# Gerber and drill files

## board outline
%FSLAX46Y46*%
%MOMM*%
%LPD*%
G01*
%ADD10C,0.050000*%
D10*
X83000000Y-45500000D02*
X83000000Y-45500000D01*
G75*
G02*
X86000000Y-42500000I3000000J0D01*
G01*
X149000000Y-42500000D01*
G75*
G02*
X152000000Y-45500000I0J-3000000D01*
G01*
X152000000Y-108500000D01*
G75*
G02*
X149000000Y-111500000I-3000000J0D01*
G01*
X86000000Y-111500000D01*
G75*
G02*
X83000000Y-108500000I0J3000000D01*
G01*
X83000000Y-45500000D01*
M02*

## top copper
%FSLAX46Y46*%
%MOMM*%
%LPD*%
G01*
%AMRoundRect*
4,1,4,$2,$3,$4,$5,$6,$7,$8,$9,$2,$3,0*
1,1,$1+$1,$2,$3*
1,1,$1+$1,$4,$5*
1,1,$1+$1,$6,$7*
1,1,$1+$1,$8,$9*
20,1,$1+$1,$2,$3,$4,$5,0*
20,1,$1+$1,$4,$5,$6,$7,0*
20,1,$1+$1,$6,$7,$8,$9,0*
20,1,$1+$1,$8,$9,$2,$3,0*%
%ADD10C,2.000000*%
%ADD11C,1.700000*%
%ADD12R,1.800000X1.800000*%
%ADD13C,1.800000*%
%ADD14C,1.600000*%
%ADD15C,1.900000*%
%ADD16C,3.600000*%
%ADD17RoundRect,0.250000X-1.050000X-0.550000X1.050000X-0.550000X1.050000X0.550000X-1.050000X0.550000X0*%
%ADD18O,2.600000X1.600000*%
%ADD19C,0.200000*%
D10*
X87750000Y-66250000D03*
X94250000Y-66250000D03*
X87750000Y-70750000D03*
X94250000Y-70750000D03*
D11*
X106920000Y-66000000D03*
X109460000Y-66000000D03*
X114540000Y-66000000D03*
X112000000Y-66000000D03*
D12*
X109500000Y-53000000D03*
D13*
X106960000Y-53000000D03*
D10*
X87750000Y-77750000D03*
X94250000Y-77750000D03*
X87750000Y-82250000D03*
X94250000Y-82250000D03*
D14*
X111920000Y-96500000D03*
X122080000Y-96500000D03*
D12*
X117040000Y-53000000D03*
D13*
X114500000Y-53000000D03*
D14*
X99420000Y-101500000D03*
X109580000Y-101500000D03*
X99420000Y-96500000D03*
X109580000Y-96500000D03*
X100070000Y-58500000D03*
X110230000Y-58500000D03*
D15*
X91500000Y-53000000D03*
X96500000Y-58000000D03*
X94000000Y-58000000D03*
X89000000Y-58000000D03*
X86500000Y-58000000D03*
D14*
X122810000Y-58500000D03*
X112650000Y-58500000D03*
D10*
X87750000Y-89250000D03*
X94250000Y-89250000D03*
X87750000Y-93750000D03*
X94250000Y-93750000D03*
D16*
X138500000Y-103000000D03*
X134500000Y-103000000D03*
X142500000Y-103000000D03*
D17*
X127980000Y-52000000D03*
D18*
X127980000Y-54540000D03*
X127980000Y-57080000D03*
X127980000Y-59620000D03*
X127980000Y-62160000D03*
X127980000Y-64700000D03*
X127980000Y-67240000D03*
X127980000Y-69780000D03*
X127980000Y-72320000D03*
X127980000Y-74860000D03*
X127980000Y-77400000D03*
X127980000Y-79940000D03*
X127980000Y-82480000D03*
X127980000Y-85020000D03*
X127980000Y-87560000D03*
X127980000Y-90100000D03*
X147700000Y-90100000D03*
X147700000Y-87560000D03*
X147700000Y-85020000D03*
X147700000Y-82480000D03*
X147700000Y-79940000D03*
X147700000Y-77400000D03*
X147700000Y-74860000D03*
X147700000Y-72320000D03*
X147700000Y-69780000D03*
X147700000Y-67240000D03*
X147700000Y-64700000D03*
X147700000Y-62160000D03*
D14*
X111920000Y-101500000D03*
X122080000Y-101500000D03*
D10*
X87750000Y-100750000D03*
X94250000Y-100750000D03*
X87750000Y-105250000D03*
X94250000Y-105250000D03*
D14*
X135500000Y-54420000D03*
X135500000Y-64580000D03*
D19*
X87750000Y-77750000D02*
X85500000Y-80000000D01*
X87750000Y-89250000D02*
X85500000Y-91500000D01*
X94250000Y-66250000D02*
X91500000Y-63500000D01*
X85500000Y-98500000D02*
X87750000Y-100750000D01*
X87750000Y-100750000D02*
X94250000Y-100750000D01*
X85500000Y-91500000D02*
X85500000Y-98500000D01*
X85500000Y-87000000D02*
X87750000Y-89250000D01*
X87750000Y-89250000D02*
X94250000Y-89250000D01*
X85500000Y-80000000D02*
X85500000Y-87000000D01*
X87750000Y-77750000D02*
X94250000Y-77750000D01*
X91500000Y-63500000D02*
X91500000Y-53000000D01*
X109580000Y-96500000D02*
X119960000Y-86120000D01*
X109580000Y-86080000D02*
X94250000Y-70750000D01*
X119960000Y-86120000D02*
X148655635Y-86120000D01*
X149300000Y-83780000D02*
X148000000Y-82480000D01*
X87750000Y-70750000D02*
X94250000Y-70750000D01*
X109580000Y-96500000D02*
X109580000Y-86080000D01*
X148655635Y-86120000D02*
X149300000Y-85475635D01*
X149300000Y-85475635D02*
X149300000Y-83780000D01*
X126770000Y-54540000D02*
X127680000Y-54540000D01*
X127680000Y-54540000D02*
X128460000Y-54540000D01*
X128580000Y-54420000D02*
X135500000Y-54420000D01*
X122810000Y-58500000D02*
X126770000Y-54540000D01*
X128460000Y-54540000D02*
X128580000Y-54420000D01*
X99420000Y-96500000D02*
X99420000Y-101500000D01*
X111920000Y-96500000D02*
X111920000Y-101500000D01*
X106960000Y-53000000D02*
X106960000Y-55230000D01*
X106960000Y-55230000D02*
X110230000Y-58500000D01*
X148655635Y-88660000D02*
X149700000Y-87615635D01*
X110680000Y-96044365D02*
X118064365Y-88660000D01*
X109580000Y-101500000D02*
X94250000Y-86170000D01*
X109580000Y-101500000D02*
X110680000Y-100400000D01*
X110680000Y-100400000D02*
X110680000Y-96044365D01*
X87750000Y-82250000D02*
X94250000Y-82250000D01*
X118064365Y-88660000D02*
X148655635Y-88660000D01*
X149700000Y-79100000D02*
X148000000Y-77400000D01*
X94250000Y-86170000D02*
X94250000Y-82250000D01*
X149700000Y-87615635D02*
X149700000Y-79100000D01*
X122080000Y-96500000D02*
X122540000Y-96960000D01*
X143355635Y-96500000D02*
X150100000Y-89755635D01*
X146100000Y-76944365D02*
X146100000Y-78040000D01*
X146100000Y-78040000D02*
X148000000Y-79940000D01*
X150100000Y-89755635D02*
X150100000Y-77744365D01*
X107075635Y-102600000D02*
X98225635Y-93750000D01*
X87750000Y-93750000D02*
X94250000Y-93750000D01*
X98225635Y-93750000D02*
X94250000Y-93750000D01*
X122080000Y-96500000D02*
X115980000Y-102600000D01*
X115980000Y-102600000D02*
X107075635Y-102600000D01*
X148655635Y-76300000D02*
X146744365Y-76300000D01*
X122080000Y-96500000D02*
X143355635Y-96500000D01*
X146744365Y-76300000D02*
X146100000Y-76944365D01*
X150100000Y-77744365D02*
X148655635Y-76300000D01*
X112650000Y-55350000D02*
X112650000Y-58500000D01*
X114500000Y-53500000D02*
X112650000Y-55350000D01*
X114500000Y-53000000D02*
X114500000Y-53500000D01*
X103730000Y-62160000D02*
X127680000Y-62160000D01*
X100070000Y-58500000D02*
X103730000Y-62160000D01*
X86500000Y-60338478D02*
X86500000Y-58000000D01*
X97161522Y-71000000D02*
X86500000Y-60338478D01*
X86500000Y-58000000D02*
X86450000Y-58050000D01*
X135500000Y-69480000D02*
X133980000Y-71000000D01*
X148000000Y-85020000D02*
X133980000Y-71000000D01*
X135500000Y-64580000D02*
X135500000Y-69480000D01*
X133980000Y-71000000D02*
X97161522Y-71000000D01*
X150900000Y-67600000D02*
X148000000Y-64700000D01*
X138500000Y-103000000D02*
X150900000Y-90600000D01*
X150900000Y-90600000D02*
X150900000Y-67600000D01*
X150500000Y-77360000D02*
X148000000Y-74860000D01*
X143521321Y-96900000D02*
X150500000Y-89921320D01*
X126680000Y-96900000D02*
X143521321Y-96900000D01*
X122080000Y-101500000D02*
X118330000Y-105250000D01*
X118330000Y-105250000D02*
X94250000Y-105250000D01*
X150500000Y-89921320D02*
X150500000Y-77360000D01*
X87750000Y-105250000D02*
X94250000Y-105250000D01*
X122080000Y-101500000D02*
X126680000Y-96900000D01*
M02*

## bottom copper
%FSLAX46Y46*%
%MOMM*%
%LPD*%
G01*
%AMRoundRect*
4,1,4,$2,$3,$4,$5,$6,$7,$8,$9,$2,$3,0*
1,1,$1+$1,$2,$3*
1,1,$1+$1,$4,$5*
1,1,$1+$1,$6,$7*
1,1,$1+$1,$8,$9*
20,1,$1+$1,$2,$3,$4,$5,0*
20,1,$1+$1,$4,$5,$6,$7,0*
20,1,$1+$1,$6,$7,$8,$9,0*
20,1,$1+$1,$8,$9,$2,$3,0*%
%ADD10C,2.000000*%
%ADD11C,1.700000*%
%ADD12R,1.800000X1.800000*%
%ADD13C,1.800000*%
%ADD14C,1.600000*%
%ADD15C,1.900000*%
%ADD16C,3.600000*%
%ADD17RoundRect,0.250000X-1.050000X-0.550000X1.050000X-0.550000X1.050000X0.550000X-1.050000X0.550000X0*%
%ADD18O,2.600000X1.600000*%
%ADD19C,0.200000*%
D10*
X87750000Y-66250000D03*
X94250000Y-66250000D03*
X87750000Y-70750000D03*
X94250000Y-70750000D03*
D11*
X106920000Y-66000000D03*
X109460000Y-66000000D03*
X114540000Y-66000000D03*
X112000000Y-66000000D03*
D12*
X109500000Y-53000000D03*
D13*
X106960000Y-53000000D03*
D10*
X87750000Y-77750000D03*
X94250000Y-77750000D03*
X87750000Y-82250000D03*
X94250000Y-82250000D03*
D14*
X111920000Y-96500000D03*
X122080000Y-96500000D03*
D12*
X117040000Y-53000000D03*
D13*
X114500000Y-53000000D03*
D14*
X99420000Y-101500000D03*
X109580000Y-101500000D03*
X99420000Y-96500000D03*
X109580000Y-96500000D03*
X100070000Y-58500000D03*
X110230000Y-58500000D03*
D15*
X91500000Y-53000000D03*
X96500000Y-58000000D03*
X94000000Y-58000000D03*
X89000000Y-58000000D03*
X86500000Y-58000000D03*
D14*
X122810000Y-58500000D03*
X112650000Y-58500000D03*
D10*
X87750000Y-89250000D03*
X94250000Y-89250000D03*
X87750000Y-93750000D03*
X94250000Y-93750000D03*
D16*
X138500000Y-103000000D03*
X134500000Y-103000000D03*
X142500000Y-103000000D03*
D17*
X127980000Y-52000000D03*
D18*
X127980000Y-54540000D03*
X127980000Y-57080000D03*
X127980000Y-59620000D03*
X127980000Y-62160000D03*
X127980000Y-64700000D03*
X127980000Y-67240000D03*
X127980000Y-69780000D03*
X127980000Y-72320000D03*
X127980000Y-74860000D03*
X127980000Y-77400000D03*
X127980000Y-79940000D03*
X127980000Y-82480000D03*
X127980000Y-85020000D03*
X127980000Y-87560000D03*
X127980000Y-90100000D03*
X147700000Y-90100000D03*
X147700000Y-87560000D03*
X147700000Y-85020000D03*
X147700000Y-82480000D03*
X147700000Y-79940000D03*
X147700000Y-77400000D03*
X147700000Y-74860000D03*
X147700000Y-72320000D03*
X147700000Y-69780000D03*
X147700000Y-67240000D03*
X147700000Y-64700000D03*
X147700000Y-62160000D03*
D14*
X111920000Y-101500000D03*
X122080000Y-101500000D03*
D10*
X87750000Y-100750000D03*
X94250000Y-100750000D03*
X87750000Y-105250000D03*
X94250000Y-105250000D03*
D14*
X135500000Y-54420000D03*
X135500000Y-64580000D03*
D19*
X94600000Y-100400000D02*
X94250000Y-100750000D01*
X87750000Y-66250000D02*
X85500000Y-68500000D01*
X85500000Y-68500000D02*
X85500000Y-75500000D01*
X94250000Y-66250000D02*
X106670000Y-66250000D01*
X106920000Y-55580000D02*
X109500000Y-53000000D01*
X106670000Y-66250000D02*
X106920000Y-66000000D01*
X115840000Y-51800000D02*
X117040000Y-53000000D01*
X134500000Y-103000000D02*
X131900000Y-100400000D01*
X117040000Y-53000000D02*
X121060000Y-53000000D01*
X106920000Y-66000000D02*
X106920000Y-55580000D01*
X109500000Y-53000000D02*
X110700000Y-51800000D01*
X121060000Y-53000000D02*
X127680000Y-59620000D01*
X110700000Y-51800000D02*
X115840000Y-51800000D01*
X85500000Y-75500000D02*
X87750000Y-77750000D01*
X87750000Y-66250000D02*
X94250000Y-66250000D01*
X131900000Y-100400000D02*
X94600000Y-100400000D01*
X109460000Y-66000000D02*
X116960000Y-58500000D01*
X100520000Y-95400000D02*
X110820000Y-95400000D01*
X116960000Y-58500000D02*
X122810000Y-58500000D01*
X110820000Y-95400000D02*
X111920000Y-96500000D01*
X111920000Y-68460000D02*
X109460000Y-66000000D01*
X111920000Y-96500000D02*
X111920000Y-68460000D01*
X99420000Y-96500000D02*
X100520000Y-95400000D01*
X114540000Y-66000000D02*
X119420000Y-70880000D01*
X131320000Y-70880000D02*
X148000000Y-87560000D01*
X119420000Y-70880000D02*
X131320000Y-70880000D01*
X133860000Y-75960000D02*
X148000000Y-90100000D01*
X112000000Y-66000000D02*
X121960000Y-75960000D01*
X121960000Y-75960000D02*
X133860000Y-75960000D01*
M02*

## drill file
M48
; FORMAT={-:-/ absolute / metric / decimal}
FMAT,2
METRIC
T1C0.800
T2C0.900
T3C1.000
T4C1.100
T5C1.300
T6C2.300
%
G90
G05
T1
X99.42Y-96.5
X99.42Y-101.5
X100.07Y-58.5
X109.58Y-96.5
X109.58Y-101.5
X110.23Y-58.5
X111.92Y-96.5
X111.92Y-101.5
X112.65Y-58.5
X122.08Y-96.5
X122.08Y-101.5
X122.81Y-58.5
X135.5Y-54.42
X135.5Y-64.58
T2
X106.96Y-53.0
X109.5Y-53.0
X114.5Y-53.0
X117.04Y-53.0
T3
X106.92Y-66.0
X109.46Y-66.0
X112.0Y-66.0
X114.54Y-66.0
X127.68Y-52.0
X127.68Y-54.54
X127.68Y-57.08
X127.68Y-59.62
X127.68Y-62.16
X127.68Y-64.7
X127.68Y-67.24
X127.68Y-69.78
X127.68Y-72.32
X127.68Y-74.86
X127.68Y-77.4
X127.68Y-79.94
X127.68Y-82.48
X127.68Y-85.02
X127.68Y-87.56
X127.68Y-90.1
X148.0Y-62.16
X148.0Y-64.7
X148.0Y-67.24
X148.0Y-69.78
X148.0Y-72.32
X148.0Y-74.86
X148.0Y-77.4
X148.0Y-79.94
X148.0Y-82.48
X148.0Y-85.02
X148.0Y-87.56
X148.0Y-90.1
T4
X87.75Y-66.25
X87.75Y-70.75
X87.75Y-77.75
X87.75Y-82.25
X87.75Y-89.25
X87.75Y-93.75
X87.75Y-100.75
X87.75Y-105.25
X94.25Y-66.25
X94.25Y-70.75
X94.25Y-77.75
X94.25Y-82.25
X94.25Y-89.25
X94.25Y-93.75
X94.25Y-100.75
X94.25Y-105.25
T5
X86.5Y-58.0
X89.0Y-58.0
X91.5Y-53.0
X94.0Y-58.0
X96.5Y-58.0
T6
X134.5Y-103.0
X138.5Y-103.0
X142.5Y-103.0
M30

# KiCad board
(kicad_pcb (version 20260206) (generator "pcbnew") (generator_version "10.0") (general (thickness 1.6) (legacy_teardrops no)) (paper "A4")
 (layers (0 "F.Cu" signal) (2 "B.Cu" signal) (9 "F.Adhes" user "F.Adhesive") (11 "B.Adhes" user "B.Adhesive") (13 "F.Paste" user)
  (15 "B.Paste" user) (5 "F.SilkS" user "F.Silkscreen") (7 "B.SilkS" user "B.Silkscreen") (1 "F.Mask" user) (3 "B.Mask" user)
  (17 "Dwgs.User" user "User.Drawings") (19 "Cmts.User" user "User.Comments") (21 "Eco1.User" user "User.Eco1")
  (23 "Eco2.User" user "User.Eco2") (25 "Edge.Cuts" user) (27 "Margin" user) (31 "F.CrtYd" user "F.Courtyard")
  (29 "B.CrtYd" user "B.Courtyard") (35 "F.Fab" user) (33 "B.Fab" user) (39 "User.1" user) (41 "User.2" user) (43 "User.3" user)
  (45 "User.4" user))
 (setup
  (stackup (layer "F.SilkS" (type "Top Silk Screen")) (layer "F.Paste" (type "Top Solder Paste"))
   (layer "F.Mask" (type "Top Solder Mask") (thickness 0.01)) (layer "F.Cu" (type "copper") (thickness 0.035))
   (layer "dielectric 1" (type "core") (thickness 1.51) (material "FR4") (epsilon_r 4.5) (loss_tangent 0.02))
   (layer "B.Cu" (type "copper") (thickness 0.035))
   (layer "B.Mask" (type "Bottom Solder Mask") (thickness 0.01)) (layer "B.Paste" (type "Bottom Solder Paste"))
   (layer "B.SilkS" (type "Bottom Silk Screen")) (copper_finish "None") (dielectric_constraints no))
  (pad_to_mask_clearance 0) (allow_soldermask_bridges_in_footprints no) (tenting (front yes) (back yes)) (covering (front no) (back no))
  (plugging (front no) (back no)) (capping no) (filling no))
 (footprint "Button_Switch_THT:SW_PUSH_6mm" (layer "F.Cu") (at 87.75 66.25)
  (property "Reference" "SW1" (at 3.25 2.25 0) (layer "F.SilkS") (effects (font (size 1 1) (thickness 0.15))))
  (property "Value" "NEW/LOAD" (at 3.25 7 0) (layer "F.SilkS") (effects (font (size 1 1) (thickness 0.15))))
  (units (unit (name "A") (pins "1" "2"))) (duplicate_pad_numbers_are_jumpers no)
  (pad "1" thru_hole circle (at 0 0 90) (size 2 2) (drill 1.1) (layers "*.Cu" "*.Mask") (remove_unused_layers no) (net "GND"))
  (pad "1" thru_hole circle (at 6.5 0 90) (size 2 2) (drill 1.1) (layers "*.Cu" "*.Mask") (remove_unused_layers no) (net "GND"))
  (pad "2" thru_hole circle (at 0 4.5 90) (size 2 2) (drill 1.1) (layers "*.Cu" "*.Mask") (remove_unused_layers no) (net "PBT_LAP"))
  (pad "2" thru_hole circle (at 6.5 4.5 90) (size 2 2) (drill 1.1) (layers "*.Cu" "*.Mask") (remove_unused_layers no) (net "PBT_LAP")))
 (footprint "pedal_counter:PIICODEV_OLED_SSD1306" (layer "F.Cu") (at 110.73 78)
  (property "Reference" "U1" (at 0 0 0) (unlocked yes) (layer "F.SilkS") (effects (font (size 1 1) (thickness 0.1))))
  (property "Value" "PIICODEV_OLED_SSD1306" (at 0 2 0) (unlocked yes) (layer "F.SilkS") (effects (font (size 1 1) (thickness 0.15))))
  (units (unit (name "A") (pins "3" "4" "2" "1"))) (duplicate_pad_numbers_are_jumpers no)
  (pad "1" thru_hole circle (at -3.81 -12) (size 1.7 1.7) (drill 1) (layers "*.Cu" "*.Mask") (remove_unused_layers no) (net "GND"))
  (pad "2" thru_hole circle (at -1.27 -12) (size 1.7 1.7) (drill 1) (layers "*.Cu" "*.Mask") (remove_unused_layers no) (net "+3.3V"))
  (pad "3" thru_hole circle (at 3.81 -12) (size 1.7 1.7) (drill 1) (layers "*.Cu" "*.Mask") (remove_unused_layers no) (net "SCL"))
  (pad "4" thru_hole circle (at 1.27 -12) (size 1.7 1.7) (drill 1) (layers "*.Cu" "*.Mask") (remove_unused_layers no) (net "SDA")))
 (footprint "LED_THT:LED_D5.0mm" (layer "F.Cu") (at 109.5 53 180)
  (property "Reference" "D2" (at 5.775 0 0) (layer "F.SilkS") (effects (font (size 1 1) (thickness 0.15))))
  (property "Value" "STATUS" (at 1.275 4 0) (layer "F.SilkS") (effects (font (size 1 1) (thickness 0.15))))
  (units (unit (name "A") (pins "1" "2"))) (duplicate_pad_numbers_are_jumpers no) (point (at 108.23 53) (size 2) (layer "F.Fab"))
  (pad "1" thru_hole rect (at 0 0 180) (size 1.8 1.8) (drill 0.9) (layers "*.Cu" "*.Mask") (remove_unused_layers no) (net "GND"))
  (pad "2" thru_hole circle (at 2.54 0 180) (size 1.8 1.8) (drill 0.9) (layers "*.Cu" "*.Mask") (remove_unused_layers no) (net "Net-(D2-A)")))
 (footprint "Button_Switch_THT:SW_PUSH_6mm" (layer "F.Cu") (at 87.75 77.75)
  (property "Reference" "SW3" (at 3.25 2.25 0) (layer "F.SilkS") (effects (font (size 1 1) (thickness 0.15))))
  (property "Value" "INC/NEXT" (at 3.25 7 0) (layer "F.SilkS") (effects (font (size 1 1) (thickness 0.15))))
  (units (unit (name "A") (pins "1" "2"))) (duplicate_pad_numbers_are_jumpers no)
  (pad "1" thru_hole circle (at 0 0 90) (size 2 2) (drill 1.1) (layers "*.Cu" "*.Mask") (remove_unused_layers no) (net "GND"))
  (pad "1" thru_hole circle (at 6.5 0 90) (size 2 2) (drill 1.1) (layers "*.Cu" "*.Mask") (remove_unused_layers no) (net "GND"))
  (pad "2" thru_hole circle (at 0 4.5 90) (size 2 2) (drill 1.1) (layers "*.Cu" "*.Mask") (remove_unused_layers no) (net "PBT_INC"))
  (pad "2" thru_hole circle (at 6.5 4.5 90) (size 2 2) (drill 1.1) (layers "*.Cu" "*.Mask") (remove_unused_layers no) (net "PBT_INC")))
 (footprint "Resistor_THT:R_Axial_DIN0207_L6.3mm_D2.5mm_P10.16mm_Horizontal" (layer "F.Cu") (at 111.92 96.5)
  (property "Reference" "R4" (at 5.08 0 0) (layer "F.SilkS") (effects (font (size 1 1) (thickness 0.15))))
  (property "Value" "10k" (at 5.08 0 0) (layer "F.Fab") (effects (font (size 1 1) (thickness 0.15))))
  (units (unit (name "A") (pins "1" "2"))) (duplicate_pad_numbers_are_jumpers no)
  (pad "1" thru_hole circle (at 0 0) (size 1.6 1.6) (drill 0.8) (layers "*.Cu" "*.Mask") (remove_unused_layers no) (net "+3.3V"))
  (pad "2" thru_hole circle (at 10.16 0) (size 1.6 1.6) (drill 0.8) (layers "*.Cu" "*.Mask") (remove_unused_layers no) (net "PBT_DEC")))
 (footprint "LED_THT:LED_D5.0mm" (layer "F.Cu") (at 117.04 53 180)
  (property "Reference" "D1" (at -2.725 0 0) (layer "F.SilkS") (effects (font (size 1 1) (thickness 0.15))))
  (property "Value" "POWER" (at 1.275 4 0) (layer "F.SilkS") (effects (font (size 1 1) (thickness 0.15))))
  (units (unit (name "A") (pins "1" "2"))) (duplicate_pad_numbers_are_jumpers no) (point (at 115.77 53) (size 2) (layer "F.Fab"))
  (pad "1" thru_hole rect (at 0 0 180) (size 1.8 1.8) (drill 0.9) (layers "*.Cu" "*.Mask") (remove_unused_layers no) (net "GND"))
  (pad "2" thru_hole circle (at 2.54 0 180) (size 1.8 1.8) (drill 0.9) (layers "*.Cu" "*.Mask") (remove_unused_layers no) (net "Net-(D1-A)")))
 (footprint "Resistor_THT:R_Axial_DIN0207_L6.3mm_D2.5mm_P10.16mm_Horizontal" (layer "F.Cu") (at 99.42 101.5)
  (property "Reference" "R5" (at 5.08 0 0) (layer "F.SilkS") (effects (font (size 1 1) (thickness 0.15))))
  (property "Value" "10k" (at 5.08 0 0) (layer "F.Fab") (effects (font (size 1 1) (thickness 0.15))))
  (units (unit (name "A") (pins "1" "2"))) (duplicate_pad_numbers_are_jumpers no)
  (pad "1" thru_hole circle (at 0 0) (size 1.6 1.6) (drill 0.8) (layers "*.Cu" "*.Mask") (remove_unused_layers no) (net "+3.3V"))
  (pad "2" thru_hole circle (at 10.16 0) (size 1.6 1.6) (drill 0.8) (layers "*.Cu" "*.Mask") (remove_unused_layers no) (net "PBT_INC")))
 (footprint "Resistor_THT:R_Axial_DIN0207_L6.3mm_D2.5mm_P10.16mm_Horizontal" (layer "F.Cu") (at 99.42 96.5)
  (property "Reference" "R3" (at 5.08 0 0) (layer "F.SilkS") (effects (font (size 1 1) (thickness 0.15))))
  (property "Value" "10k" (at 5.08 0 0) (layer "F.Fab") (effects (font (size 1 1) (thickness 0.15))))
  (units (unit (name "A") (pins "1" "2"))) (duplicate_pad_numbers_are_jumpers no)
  (pad "1" thru_hole circle (at 0 0) (size 1.6 1.6) (drill 0.8) (layers "*.Cu" "*.Mask") (remove_unused_layers no) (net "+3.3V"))
  (pad "2" thru_hole circle (at 10.16 0) (size 1.6 1.6) (drill 0.8) (layers "*.Cu" "*.Mask") (remove_unused_layers no) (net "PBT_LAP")))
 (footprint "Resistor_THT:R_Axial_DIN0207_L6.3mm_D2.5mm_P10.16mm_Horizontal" (layer "F.Cu") (at 100.07 58.5)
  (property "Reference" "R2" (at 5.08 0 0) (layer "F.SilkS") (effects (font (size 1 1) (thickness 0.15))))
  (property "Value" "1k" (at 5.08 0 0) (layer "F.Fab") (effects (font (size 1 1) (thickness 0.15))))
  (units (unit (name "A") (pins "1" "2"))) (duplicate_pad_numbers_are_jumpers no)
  (pad "1" thru_hole circle (at 0 0) (size 1.6 1.6) (drill 0.8) (layers "*.Cu" "*.Mask") (remove_unused_layers no) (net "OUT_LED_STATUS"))
  (pad "2" thru_hole circle (at 10.16 0) (size 1.6 1.6) (drill 0.8) (layers "*.Cu" "*.Mask") (remove_unused_layers no) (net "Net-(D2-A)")))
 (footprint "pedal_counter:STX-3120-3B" (layer "F.Cu") (at 91.5 58 -90)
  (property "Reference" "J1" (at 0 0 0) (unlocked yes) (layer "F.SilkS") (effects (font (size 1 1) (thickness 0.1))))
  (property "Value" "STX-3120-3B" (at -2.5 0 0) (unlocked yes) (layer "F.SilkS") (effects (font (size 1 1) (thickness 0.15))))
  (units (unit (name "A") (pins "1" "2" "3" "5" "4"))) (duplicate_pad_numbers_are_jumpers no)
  (pad "1" thru_hole circle (at -5 0 270) (size 1.9 1.9) (drill 1.3) (layers "*.Cu" "*.Mask") (remove_unused_layers no) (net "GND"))
  (pad "2" thru_hole circle (at 0 -5 270) (size 1.9 1.9) (drill 1.3) (layers "*.Cu" "*.Mask") (remove_unused_layers no)
   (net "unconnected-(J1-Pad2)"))
  (pad "3" thru_hole circle (at 0 -2.5 270) (size 1.9 1.9) (drill 1.3) (layers "*.Cu" "*.Mask") (remove_unused_layers no)
   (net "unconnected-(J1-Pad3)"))
  (pad "4" thru_hole circle (at 0 2.5 270) (size 1.9 1.9) (drill 1.3) (layers "*.Cu" "*.Mask") (remove_unused_layers no)
   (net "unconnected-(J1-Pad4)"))
  (pad "5" thru_hole circle (at 0 5 270) (size 1.9 1.9) (drill 1.3) (layers "*.Cu" "*.Mask") (remove_unused_layers no) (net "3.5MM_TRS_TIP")))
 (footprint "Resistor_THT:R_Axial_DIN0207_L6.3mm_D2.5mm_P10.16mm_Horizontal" (layer "F.Cu") (at 122.81 58.5 180)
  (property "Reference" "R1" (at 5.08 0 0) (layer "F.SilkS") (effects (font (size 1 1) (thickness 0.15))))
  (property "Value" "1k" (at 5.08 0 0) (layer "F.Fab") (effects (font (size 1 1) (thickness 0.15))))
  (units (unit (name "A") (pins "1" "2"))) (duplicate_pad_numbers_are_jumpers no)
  (pad "1" thru_hole circle (at 0 0 180) (size 1.6 1.6) (drill 0.8) (layers "*.Cu" "*.Mask") (remove_unused_layers no) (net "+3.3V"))
  (pad "2" thru_hole circle (at 10.16 0 180) (size 1.6 1.6) (drill 0.8) (layers "*.Cu" "*.Mask") (remove_unused_layers no)
   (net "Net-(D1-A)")))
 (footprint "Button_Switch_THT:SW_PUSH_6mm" (layer "F.Cu") (at 87.75 89.25)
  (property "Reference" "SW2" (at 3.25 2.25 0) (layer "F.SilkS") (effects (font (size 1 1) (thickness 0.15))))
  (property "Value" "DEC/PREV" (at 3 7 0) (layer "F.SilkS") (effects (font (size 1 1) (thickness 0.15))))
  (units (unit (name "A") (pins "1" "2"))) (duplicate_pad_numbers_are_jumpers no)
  (pad "1" thru_hole circle (at 0 0 90) (size 2 2) (drill 1.1) (layers "*.Cu" "*.Mask") (remove_unused_layers no) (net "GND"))
  (pad "1" thru_hole circle (at 6.5 0 90) (size 2 2) (drill 1.1) (layers "*.Cu" "*.Mask") (remove_unused_layers no) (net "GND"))
  (pad "2" thru_hole circle (at 0 4.5 90) (size 2 2) (drill 1.1) (layers "*.Cu" "*.Mask") (remove_unused_layers no) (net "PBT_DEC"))
  (pad "2" thru_hole circle (at 6.5 4.5 90) (size 2 2) (drill 1.1) (layers "*.Cu" "*.Mask") (remove_unused_layers no) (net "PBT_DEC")))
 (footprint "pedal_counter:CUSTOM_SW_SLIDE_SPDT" (layer "F.Cu") (at 138.5 103)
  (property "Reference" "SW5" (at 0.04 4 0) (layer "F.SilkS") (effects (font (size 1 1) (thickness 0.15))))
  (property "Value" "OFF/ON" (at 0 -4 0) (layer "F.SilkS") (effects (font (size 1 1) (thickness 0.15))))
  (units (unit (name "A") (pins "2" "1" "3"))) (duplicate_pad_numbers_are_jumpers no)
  (pad "1" thru_hole circle (at 0 0) (size 3.6 3.6) (drill 2.3) (layers "*.Cu" "*.Mask") (remove_unused_layers no) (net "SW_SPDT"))
  (pad "2" thru_hole circle (at -4 0) (size 3.6 3.6) (drill 2.3) (layers "*.Cu" "*.Mask") (remove_unused_layers no) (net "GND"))
  (pad "3" thru_hole circle (at 4 0) (size 3.6 3.6) (drill 2.3) (layers "*.Cu" "*.Mask") (remove_unused_layers no)
   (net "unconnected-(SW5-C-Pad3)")))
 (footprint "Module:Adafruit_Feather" (layer "F.Cu") (at 127.68 52)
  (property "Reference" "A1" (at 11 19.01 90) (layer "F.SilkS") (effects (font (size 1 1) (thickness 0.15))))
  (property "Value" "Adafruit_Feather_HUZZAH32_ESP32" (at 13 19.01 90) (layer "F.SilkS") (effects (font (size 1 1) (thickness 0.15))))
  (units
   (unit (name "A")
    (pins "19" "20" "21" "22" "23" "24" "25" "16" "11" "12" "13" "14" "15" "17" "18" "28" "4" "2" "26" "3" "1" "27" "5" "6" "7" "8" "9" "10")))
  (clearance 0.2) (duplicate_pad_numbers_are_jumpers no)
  (pad "1" thru_hole roundrect (at 0 0) (size 2.6 1.6) (drill 1 (offset 0.3 0)) (layers "*.Cu" "*.Mask") (remove_unused_layers no)
   (roundrect_rratio 0.15625) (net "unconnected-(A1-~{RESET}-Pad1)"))
  (pad "2" thru_hole oval (at 0 2.54) (size 2.6 1.6) (drill 1 (offset 0.3 0)) (layers "*.Cu" "*.Mask") (remove_unused_layers no)
   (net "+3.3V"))
  (pad "3" thru_hole oval (at 0 5.08) (size 2.6 1.6) (drill 1 (offset 0.3 0)) (layers "*.Cu" "*.Mask") (remove_unused_layers no)
   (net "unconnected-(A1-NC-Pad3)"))
  (pad "4" thru_hole oval (at 0 7.62) (size 2.6 1.6) (drill 1 (offset 0.3 0)) (layers "*.Cu" "*.Mask") (remove_unused_layers no) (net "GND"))
  (pad "5" thru_hole oval (at 0 10.16) (size 2.6 1.6) (drill 1 (offset 0.3 0)) (layers "*.Cu" "*.Mask") (remove_unused_layers no)
   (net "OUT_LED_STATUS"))
  (pad "6" thru_hole oval (at 0 12.7) (size 2.6 1.6) (drill 1 (offset 0.3 0)) (layers "*.Cu" "*.Mask") (remove_unused_layers no)
   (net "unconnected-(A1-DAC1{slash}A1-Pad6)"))
  (pad "7" thru_hole oval (at 0 15.24) (size 2.6 1.6) (drill 1 (offset 0.3 0)) (layers "*.Cu" "*.Mask") (remove_unused_layers no)
   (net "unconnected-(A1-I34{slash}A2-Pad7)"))
  (pad "8" thru_hole oval (at 0 17.78) (size 2.6 1.6) (drill 1 (offset 0.3 0)) (layers "*.Cu" "*.Mask") (remove_unused_layers no)
   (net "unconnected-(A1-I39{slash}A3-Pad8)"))
  (pad "9" thru_hole oval (at 0 20.32) (size 2.6 1.6) (drill 1 (offset 0.3 0)) (layers "*.Cu" "*.Mask") (remove_unused_layers no)
   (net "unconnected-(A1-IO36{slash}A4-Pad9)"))
  (pad "10" thru_hole oval (at 0 22.86) (size 2.6 1.6) (drill 1 (offset 0.3 0)) (layers "*.Cu" "*.Mask") (remove_unused_layers no)
   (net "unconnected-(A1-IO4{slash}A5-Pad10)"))
  (pad "11" thru_hole oval (at 0 25.4) (size 2.6 1.6) (drill 1 (offset 0.3 0)) (layers "*.Cu" "*.Mask") (remove_unused_layers no)
   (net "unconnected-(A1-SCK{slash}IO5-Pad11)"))
  (pad "12" thru_hole oval (at 0 27.94) (size 2.6 1.6) (drill 1 (offset 0.3 0)) (layers "*.Cu" "*.Mask") (remove_unused_layers no)
   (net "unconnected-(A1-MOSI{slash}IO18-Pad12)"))
  (pad "13" thru_hole oval (at 0 30.48) (size 2.6 1.6) (drill 1 (offset 0.3 0)) (layers "*.Cu" "*.Mask") (remove_unused_layers no)
   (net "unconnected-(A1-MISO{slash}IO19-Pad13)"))
  (pad "14" thru_hole oval (at 0 33.02) (size 2.6 1.6) (drill 1 (offset 0.3 0)) (layers "*.Cu" "*.Mask") (remove_unused_layers no)
   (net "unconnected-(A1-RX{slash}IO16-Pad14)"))
  (pad "15" thru_hole oval (at 0 35.56) (size 2.6 1.6) (drill 1 (offset 0.3 0)) (layers "*.Cu" "*.Mask") (remove_unused_layers no)
   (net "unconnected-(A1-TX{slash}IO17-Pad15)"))
  (pad "16" thru_hole oval (at 0 38.1) (size 2.6 1.6) (drill 1 (offset 0.3 0)) (layers "*.Cu" "*.Mask") (remove_unused_layers no)
   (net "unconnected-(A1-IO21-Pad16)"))
  (pad "17" thru_hole oval (at 20.32 38.1 180) (size 2.6 1.6) (drill 1 (offset 0.3 0)) (layers "*.Cu" "*.Mask") (remove_unused_layers no)
   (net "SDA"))
  (pad "18" thru_hole oval (at 20.32 35.56 180) (size 2.6 1.6) (drill 1 (offset 0.3 0)) (layers "*.Cu" "*.Mask") (remove_unused_layers no)
   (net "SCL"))
  (pad "19" thru_hole oval (at 20.32 33.02 180) (size 2.6 1.6) (drill 1 (offset 0.3 0)) (layers "*.Cu" "*.Mask") (remove_unused_layers no)
   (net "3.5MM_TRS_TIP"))
  (pad "20" thru_hole oval (at 20.32 30.48 180) (size 2.6 1.6) (drill 1 (offset 0.3 0)) (layers "*.Cu" "*.Mask") (remove_unused_layers no)
   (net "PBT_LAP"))
  (pad "21" thru_hole oval (at 20.32 27.94 180) (size 2.6 1.6) (drill 1 (offset 0.3 0)) (layers "*.Cu" "*.Mask") (remove_unused_layers no)
   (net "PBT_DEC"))
  (pad "22" thru_hole oval (at 20.32 25.4 180) (size 2.6 1.6) (drill 1 (offset 0.3 0)) (layers "*.Cu" "*.Mask") (remove_unused_layers no)
   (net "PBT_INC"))
  (pad "23" thru_hole oval (at 20.32 22.86 180) (size 2.6 1.6) (drill 1 (offset 0.3 0)) (layers "*.Cu" "*.Mask") (remove_unused_layers no)
   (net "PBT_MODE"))
  (pad "24" thru_hole oval (at 20.32 20.32 180) (size 2.6 1.6) (drill 1 (offset 0.3 0)) (layers "*.Cu" "*.Mask") (remove_unused_layers no)
   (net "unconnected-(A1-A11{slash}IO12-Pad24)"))
  (pad "25" thru_hole oval (at 20.32 17.78 180) (size 2.6 1.6) (drill 1 (offset 0.3 0)) (layers "*.Cu" "*.Mask") (remove_unused_layers no)
   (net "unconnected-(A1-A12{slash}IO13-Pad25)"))
  (pad "26" thru_hole oval (at 20.32 15.24 180) (size 2.6 1.6) (drill 1 (offset 0.3 0)) (layers "*.Cu" "*.Mask") (remove_unused_layers no)
   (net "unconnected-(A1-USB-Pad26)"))
  (pad "27" thru_hole oval (at 20.32 12.7 180) (size 2.6 1.6) (drill 1 (offset 0.3 0)) (layers "*.Cu" "*.Mask") (remove_unused_layers no)
   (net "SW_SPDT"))
  (pad "28" thru_hole oval (at 20.32 10.16 180) (size 2.6 1.6) (drill 1 (offset 0.3 0)) (layers "*.Cu" "*.Mask") (remove_unused_layers no)
   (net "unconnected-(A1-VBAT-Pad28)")))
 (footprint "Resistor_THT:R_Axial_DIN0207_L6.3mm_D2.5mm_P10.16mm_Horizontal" (layer "F.Cu") (at 111.92 101.5)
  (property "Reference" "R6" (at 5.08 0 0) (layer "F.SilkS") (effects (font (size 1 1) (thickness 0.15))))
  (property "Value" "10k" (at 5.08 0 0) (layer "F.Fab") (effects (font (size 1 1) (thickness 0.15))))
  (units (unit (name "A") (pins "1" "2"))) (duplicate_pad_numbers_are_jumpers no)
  (pad "1" thru_hole circle (at 0 0) (size 1.6 1.6) (drill 0.8) (layers "*.Cu" "*.Mask") (remove_unused_layers no) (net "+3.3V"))
  (pad "2" thru_hole circle (at 10.16 0) (size 1.6 1.6) (drill 0.8) (layers "*.Cu" "*.Mask") (remove_unused_layers no) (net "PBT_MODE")))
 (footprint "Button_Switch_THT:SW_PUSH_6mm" (layer "F.Cu") (at 87.75 100.75)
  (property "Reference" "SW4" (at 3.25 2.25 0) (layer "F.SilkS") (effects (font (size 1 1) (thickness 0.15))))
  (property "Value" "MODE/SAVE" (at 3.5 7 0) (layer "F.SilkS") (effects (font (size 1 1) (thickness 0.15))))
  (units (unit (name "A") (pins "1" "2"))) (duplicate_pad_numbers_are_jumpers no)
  (pad "1" thru_hole circle (at 0 0 90) (size 2 2) (drill 1.1) (layers "*.Cu" "*.Mask") (remove_unused_layers no) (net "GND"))
  (pad "1" thru_hole circle (at 6.5 0 90) (size 2 2) (drill 1.1) (layers "*.Cu" "*.Mask") (remove_unused_layers no) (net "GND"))
  (pad "2" thru_hole circle (at 0 4.5 90) (size 2 2) (drill 1.1) (layers "*.Cu" "*.Mask") (remove_unused_layers no) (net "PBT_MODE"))
  (pad "2" thru_hole circle (at 6.5 4.5 90) (size 2 2) (drill 1.1) (layers "*.Cu" "*.Mask") (remove_unused_layers no) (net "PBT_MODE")))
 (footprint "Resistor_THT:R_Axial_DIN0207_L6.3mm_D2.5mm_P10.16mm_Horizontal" (layer "B.Cu") (at 135.5 54.42 -90)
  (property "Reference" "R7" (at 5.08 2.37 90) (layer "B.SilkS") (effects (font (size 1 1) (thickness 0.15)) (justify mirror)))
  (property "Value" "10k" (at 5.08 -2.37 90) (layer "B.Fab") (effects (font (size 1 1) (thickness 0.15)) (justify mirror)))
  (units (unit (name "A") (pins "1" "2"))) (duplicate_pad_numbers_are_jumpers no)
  (pad "1" thru_hole circle (at 0 0 270) (size 1.6 1.6) (drill 0.8) (layers "*.Cu" "*.Mask") (remove_unused_layers no) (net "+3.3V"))
  (pad "2" thru_hole circle (at 10.16 0 270) (size 1.6 1.6) (drill 0.8) (layers "*.Cu" "*.Mask") (remove_unused_layers no)
   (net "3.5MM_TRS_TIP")))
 (gr_rect (start 83 42.5) (end 152 111.5) (radius 3) (stroke (width 0.05) (type solid)) (fill no) (layer "Edge.Cuts"))
 (segment (start 87.75 77.75) (end 85.5 80) (width 0.2) (layer "F.Cu") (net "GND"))
 (segment (start 87.75 89.25) (end 85.5 91.5) (width 0.2) (layer "F.Cu") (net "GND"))
 (segment (start 94.25 66.25) (end 91.5 63.5) (width 0.2) (layer "F.Cu") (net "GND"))
 (segment (start 85.5 98.5) (end 87.75 100.75) (width 0.2) (layer "F.Cu") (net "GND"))
 (segment (start 87.75 100.75) (end 94.25 100.75) (width 0.2) (layer "F.Cu") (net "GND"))
 (segment (start 85.5 91.5) (end 85.5 98.5) (width 0.2) (layer "F.Cu") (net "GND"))
 (segment (start 85.5 87) (end 87.75 89.25) (width 0.2) (layer "F.Cu") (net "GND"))
 (segment (start 87.75 89.25) (end 94.25 89.25) (width 0.2) (layer "F.Cu") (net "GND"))
 (segment (start 85.5 80) (end 85.5 87) (width 0.2) (layer "F.Cu") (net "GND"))
 (segment (start 87.75 77.75) (end 94.25 77.75) (width 0.2) (layer "F.Cu") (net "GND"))
 (segment (start 91.5 63.5) (end 91.5 53) (width 0.2) (layer "F.Cu") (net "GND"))
 (segment (start 94.6 100.4) (end 94.25 100.75) (width 0.2) (layer "B.Cu") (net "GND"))
 (segment (start 87.75 66.25) (end 85.5 68.5) (width 0.2) (layer "B.Cu") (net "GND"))
 (segment (start 85.5 68.5) (end 85.5 75.5) (width 0.2) (layer "B.Cu") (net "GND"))
 (segment (start 94.25 66.25) (end 106.67 66.25) (width 0.2) (layer "B.Cu") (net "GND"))
 (segment (start 106.92 55.58) (end 109.5 53) (width 0.2) (layer "B.Cu") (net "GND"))
 (segment (start 106.67 66.25) (end 106.92 66) (width 0.2) (layer "B.Cu") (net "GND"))
 (segment (start 115.84 51.8) (end 117.04 53) (width 0.2) (layer "B.Cu") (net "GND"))
 (segment (start 134.5 103) (end 131.9 100.4) (width 0.2) (layer "B.Cu") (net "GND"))
 (segment (start 117.04 53) (end 121.06 53) (width 0.2) (layer "B.Cu") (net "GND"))
 (segment (start 106.92 66) (end 106.92 55.58) (width 0.2) (layer "B.Cu") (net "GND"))
 (segment (start 109.5 53) (end 110.7 51.8) (width 0.2) (layer "B.Cu") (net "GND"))
 (segment (start 121.06 53) (end 127.68 59.62) (width 0.2) (layer "B.Cu") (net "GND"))
 (segment (start 110.7 51.8) (end 115.84 51.8) (width 0.2) (layer "B.Cu") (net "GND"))
 (segment (start 85.5 75.5) (end 87.75 77.75) (width 0.2) (layer "B.Cu") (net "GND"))
 (segment (start 87.75 66.25) (end 94.25 66.25) (width 0.2) (layer "B.Cu") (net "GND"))
 (segment (start 131.9 100.4) (end 94.6 100.4) (width 0.2) (layer "B.Cu") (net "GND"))
 (segment (start 109.58 96.5) (end 119.96 86.12) (width 0.2) (layer "F.Cu") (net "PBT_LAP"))
 (segment (start 109.58 86.08) (end 94.25 70.75) (width 0.2) (layer "F.Cu") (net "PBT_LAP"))
 (segment (start 119.96 86.12) (end 148.655635 86.12) (width 0.2) (layer "F.Cu") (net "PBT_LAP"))
 (segment (start 149.3 83.78) (end 148 82.48) (width 0.2) (layer "F.Cu") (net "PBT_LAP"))
 (segment (start 87.75 70.75) (end 94.25 70.75) (width 0.2) (layer "F.Cu") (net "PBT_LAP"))
 (segment (start 109.58 96.5) (end 109.58 86.08) (width 0.2) (layer "F.Cu") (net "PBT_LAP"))
 (segment (start 148.655635 86.12) (end 149.3 85.475635) (width 0.2) (layer "F.Cu") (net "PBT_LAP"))
 (segment (start 149.3 85.475635) (end 149.3 83.78) (width 0.2) (layer "F.Cu") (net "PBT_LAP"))
 (segment (start 126.77 54.54) (end 127.68 54.54) (width 0.2) (layer "F.Cu") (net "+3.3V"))
 (segment (start 127.68 54.54) (end 128.46 54.54) (width 0.2) (layer "F.Cu") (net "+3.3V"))
 (segment (start 128.58 54.42) (end 135.5 54.42) (width 0.2) (layer "F.Cu") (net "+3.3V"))
 (segment (start 122.81 58.5) (end 126.77 54.54) (width 0.2) (layer "F.Cu") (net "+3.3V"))
 (segment (start 128.46 54.54) (end 128.58 54.42) (width 0.2) (layer "F.Cu") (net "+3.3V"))
 (segment (start 99.42 96.5) (end 99.42 101.5) (width 0.2) (layer "F.Cu") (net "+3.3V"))
 (segment (start 111.92 96.5) (end 111.92 101.5) (width 0.2) (layer "F.Cu") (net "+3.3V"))
 (segment (start 109.46 66) (end 116.96 58.5) (width 0.2) (layer "B.Cu") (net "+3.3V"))
 (segment (start 100.52 95.4) (end 110.82 95.4) (width 0.2) (layer "B.Cu") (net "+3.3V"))
 (segment (start 116.96 58.5) (end 122.81 58.5) (width 0.2) (layer "B.Cu") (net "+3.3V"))
 (segment (start 110.82 95.4) (end 111.92 96.5) (width 0.2) (layer "B.Cu") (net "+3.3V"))
 (segment (start 111.92 68.46) (end 109.46 66) (width 0.2) (layer "B.Cu") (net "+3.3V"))
 (segment (start 111.92 96.5) (end 111.92 68.46) (width 0.2) (layer "B.Cu") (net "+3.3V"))
 (segment (start 99.42 96.5) (end 100.52 95.4) (width 0.2) (layer "B.Cu") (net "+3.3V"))
 (segment (start 114.54 66) (end 119.42 70.88) (width 0.2) (layer "B.Cu") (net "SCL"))
 (segment (start 131.32 70.88) (end 148 87.56) (width 0.2) (layer "B.Cu") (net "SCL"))
 (segment (start 119.42 70.88) (end 131.32 70.88) (width 0.2) (layer "B.Cu") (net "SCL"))
 (segment (start 133.86 75.96) (end 148 90.1) (width 0.2) (layer "B.Cu") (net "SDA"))
 (segment (start 112 66) (end 121.96 75.96) (width 0.2) (layer "B.Cu") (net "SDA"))
 (segment (start 121.96 75.96) (end 133.86 75.96) (width 0.2) (layer "B.Cu") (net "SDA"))
 (segment (start 106.96 53) (end 106.96 55.23) (width 0.2) (layer "F.Cu") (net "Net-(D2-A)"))
 (segment (start 106.96 55.23) (end 110.23 58.5) (width 0.2) (layer "F.Cu") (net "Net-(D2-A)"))
 (segment (start 148.655635 88.66) (end 149.7 87.615635) (width 0.2) (layer "F.Cu") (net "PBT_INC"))
 (segment (start 110.68 96.044365) (end 118.064365 88.66) (width 0.2) (layer "F.Cu") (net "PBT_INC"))
 (segment (start 109.58 101.5) (end 94.25 86.17) (width 0.2) (layer "F.Cu") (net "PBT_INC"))
 (segment (start 109.58 101.5) (end 110.68 100.4) (width 0.2) (layer "F.Cu") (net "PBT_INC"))
 (segment (start 110.68 100.4) (end 110.68 96.044365) (width 0.2) (layer "F.Cu") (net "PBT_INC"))
 (segment (start 87.75 82.25) (end 94.25 82.25) (width 0.2) (layer "F.Cu") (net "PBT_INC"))
 (segment (start 118.064365 88.66) (end 148.655635 88.66) (width 0.2) (layer "F.Cu") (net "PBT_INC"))
 (segment (start 149.7 79.1) (end 148 77.4) (width 0.2) (layer "F.Cu") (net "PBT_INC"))
 (segment (start 94.25 86.17) (end 94.25 82.25) (width 0.2) (layer "F.Cu") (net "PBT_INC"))
 (segment (start 149.7 87.615635) (end 149.7 79.1) (width 0.2) (layer "F.Cu") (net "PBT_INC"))
 (segment (start 122.08 96.5) (end 122.54 96.96) (width 0.2) (layer "F.Cu") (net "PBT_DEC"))
 (segment (start 143.355635 96.5) (end 150.1 89.755635) (width 0.2) (layer "F.Cu") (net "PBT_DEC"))
 (segment (start 146.1 76.944365) (end 146.1 78.04) (width 0.2) (layer "F.Cu") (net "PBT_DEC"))
 (segment (start 146.1 78.04) (end 148 79.94) (width 0.2) (layer "F.Cu") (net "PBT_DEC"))
 (segment (start 150.1 89.755635) (end 150.1 77.744365) (width 0.2) (layer "F.Cu") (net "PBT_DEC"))
 (segment (start 107.075635 102.6) (end 98.225635 93.75) (width 0.2) (layer "F.Cu") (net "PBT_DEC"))
 (segment (start 87.75 93.75) (end 94.25 93.75) (width 0.2) (layer "F.Cu") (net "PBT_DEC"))
 (segment (start 98.225635 93.75) (end 94.25 93.75) (width 0.2) (layer "F.Cu") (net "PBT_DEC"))
 (segment (start 122.08 96.5) (end 115.98 102.6) (width 0.2) (layer "F.Cu") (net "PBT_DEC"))
 (segment (start 115.98 102.6) (end 107.075635 102.6) (width 0.2) (layer "F.Cu") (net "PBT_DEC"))
 (segment (start 148.655635 76.3) (end 146.744365 76.3) (width 0.2) (layer "F.Cu") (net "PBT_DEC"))
 (segment (start 122.08 96.5) (end 143.355635 96.5) (width 0.2) (layer "F.Cu") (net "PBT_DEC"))
 (segment (start 146.744365 76.3) (end 146.1 76.944365) (width 0.2) (layer "F.Cu") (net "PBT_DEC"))
 (segment (start 150.1 77.744365) (end 148.655635 76.3) (width 0.2) (layer "F.Cu") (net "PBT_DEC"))
 (segment (start 112.65 55.35) (end 112.65 58.5) (width 0.2) (layer "F.Cu") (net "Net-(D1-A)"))
 (segment (start 114.5 53.5) (end 112.65 55.35) (width 0.2) (layer "F.Cu") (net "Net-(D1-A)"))
 (segment (start 114.5 53) (end 114.5 53.5) (width 0.2) (layer "F.Cu") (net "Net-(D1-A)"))
 (segment (start 103.73 62.16) (end 127.68 62.16) (width 0.2) (layer "F.Cu") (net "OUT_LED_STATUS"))
 (segment (start 100.07 58.5) (end 103.73 62.16) (width 0.2) (layer "F.Cu") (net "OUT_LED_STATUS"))
 (segment (start 86.5 60.338478) (end 86.5 58) (width 0.2) (layer "F.Cu") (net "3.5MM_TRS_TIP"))
 (segment (start 97.161522 71) (end 86.5 60.338478) (width 0.2) (layer "F.Cu") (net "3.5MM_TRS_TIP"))
 (segment (start 86.5 58) (end 86.45 58.05) (width 0.2) (layer "F.Cu") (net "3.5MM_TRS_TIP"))
 (segment (start 135.5 69.48) (end 133.98 71) (width 0.2) (layer "F.Cu") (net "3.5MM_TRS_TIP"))
 (segment (start 148 85.02) (end 133.98 71) (width 0.2) (layer "F.Cu") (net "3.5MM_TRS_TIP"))
 (segment (start 135.5 64.58) (end 135.5 69.48) (width 0.2) (layer "F.Cu") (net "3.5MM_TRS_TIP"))
 (segment (start 133.98 71) (end 97.161522 71) (width 0.2) (layer "F.Cu") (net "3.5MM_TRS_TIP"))
 (segment (start 150.9 67.6) (end 148 64.7) (width 0.2) (layer "F.Cu") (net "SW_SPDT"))
 (segment (start 138.5 103) (end 150.9 90.6) (width 0.2) (layer "F.Cu") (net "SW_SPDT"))
 (segment (start 150.9 90.6) (end 150.9 67.6) (width 0.2) (layer "F.Cu") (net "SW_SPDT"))
 (segment (start 150.5 77.36) (end 148 74.86) (width 0.2) (layer "F.Cu") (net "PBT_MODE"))
 (segment (start 143.521321 96.9) (end 150.5 89.92132) (width 0.2) (layer "F.Cu") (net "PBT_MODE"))
 (segment (start 126.68 96.9) (end 143.521321 96.9) (width 0.2) (layer "F.Cu") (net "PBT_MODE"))
 (segment (start 122.08 101.5) (end 118.33 105.25) (width 0.2) (layer "F.Cu") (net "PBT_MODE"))
 (segment (start 118.33 105.25) (end 94.25 105.25) (width 0.2) (layer "F.Cu") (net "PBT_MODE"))
 (segment (start 150.5 89.92132) (end 150.5 77.36) (width 0.2) (layer "F.Cu") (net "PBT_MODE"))
 (segment (start 87.75 105.25) (end 94.25 105.25) (width 0.2) (layer "F.Cu") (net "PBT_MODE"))
 (segment (start 122.08 101.5) (end 126.68 96.9) (width 0.2) (layer "F.Cu") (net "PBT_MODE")))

